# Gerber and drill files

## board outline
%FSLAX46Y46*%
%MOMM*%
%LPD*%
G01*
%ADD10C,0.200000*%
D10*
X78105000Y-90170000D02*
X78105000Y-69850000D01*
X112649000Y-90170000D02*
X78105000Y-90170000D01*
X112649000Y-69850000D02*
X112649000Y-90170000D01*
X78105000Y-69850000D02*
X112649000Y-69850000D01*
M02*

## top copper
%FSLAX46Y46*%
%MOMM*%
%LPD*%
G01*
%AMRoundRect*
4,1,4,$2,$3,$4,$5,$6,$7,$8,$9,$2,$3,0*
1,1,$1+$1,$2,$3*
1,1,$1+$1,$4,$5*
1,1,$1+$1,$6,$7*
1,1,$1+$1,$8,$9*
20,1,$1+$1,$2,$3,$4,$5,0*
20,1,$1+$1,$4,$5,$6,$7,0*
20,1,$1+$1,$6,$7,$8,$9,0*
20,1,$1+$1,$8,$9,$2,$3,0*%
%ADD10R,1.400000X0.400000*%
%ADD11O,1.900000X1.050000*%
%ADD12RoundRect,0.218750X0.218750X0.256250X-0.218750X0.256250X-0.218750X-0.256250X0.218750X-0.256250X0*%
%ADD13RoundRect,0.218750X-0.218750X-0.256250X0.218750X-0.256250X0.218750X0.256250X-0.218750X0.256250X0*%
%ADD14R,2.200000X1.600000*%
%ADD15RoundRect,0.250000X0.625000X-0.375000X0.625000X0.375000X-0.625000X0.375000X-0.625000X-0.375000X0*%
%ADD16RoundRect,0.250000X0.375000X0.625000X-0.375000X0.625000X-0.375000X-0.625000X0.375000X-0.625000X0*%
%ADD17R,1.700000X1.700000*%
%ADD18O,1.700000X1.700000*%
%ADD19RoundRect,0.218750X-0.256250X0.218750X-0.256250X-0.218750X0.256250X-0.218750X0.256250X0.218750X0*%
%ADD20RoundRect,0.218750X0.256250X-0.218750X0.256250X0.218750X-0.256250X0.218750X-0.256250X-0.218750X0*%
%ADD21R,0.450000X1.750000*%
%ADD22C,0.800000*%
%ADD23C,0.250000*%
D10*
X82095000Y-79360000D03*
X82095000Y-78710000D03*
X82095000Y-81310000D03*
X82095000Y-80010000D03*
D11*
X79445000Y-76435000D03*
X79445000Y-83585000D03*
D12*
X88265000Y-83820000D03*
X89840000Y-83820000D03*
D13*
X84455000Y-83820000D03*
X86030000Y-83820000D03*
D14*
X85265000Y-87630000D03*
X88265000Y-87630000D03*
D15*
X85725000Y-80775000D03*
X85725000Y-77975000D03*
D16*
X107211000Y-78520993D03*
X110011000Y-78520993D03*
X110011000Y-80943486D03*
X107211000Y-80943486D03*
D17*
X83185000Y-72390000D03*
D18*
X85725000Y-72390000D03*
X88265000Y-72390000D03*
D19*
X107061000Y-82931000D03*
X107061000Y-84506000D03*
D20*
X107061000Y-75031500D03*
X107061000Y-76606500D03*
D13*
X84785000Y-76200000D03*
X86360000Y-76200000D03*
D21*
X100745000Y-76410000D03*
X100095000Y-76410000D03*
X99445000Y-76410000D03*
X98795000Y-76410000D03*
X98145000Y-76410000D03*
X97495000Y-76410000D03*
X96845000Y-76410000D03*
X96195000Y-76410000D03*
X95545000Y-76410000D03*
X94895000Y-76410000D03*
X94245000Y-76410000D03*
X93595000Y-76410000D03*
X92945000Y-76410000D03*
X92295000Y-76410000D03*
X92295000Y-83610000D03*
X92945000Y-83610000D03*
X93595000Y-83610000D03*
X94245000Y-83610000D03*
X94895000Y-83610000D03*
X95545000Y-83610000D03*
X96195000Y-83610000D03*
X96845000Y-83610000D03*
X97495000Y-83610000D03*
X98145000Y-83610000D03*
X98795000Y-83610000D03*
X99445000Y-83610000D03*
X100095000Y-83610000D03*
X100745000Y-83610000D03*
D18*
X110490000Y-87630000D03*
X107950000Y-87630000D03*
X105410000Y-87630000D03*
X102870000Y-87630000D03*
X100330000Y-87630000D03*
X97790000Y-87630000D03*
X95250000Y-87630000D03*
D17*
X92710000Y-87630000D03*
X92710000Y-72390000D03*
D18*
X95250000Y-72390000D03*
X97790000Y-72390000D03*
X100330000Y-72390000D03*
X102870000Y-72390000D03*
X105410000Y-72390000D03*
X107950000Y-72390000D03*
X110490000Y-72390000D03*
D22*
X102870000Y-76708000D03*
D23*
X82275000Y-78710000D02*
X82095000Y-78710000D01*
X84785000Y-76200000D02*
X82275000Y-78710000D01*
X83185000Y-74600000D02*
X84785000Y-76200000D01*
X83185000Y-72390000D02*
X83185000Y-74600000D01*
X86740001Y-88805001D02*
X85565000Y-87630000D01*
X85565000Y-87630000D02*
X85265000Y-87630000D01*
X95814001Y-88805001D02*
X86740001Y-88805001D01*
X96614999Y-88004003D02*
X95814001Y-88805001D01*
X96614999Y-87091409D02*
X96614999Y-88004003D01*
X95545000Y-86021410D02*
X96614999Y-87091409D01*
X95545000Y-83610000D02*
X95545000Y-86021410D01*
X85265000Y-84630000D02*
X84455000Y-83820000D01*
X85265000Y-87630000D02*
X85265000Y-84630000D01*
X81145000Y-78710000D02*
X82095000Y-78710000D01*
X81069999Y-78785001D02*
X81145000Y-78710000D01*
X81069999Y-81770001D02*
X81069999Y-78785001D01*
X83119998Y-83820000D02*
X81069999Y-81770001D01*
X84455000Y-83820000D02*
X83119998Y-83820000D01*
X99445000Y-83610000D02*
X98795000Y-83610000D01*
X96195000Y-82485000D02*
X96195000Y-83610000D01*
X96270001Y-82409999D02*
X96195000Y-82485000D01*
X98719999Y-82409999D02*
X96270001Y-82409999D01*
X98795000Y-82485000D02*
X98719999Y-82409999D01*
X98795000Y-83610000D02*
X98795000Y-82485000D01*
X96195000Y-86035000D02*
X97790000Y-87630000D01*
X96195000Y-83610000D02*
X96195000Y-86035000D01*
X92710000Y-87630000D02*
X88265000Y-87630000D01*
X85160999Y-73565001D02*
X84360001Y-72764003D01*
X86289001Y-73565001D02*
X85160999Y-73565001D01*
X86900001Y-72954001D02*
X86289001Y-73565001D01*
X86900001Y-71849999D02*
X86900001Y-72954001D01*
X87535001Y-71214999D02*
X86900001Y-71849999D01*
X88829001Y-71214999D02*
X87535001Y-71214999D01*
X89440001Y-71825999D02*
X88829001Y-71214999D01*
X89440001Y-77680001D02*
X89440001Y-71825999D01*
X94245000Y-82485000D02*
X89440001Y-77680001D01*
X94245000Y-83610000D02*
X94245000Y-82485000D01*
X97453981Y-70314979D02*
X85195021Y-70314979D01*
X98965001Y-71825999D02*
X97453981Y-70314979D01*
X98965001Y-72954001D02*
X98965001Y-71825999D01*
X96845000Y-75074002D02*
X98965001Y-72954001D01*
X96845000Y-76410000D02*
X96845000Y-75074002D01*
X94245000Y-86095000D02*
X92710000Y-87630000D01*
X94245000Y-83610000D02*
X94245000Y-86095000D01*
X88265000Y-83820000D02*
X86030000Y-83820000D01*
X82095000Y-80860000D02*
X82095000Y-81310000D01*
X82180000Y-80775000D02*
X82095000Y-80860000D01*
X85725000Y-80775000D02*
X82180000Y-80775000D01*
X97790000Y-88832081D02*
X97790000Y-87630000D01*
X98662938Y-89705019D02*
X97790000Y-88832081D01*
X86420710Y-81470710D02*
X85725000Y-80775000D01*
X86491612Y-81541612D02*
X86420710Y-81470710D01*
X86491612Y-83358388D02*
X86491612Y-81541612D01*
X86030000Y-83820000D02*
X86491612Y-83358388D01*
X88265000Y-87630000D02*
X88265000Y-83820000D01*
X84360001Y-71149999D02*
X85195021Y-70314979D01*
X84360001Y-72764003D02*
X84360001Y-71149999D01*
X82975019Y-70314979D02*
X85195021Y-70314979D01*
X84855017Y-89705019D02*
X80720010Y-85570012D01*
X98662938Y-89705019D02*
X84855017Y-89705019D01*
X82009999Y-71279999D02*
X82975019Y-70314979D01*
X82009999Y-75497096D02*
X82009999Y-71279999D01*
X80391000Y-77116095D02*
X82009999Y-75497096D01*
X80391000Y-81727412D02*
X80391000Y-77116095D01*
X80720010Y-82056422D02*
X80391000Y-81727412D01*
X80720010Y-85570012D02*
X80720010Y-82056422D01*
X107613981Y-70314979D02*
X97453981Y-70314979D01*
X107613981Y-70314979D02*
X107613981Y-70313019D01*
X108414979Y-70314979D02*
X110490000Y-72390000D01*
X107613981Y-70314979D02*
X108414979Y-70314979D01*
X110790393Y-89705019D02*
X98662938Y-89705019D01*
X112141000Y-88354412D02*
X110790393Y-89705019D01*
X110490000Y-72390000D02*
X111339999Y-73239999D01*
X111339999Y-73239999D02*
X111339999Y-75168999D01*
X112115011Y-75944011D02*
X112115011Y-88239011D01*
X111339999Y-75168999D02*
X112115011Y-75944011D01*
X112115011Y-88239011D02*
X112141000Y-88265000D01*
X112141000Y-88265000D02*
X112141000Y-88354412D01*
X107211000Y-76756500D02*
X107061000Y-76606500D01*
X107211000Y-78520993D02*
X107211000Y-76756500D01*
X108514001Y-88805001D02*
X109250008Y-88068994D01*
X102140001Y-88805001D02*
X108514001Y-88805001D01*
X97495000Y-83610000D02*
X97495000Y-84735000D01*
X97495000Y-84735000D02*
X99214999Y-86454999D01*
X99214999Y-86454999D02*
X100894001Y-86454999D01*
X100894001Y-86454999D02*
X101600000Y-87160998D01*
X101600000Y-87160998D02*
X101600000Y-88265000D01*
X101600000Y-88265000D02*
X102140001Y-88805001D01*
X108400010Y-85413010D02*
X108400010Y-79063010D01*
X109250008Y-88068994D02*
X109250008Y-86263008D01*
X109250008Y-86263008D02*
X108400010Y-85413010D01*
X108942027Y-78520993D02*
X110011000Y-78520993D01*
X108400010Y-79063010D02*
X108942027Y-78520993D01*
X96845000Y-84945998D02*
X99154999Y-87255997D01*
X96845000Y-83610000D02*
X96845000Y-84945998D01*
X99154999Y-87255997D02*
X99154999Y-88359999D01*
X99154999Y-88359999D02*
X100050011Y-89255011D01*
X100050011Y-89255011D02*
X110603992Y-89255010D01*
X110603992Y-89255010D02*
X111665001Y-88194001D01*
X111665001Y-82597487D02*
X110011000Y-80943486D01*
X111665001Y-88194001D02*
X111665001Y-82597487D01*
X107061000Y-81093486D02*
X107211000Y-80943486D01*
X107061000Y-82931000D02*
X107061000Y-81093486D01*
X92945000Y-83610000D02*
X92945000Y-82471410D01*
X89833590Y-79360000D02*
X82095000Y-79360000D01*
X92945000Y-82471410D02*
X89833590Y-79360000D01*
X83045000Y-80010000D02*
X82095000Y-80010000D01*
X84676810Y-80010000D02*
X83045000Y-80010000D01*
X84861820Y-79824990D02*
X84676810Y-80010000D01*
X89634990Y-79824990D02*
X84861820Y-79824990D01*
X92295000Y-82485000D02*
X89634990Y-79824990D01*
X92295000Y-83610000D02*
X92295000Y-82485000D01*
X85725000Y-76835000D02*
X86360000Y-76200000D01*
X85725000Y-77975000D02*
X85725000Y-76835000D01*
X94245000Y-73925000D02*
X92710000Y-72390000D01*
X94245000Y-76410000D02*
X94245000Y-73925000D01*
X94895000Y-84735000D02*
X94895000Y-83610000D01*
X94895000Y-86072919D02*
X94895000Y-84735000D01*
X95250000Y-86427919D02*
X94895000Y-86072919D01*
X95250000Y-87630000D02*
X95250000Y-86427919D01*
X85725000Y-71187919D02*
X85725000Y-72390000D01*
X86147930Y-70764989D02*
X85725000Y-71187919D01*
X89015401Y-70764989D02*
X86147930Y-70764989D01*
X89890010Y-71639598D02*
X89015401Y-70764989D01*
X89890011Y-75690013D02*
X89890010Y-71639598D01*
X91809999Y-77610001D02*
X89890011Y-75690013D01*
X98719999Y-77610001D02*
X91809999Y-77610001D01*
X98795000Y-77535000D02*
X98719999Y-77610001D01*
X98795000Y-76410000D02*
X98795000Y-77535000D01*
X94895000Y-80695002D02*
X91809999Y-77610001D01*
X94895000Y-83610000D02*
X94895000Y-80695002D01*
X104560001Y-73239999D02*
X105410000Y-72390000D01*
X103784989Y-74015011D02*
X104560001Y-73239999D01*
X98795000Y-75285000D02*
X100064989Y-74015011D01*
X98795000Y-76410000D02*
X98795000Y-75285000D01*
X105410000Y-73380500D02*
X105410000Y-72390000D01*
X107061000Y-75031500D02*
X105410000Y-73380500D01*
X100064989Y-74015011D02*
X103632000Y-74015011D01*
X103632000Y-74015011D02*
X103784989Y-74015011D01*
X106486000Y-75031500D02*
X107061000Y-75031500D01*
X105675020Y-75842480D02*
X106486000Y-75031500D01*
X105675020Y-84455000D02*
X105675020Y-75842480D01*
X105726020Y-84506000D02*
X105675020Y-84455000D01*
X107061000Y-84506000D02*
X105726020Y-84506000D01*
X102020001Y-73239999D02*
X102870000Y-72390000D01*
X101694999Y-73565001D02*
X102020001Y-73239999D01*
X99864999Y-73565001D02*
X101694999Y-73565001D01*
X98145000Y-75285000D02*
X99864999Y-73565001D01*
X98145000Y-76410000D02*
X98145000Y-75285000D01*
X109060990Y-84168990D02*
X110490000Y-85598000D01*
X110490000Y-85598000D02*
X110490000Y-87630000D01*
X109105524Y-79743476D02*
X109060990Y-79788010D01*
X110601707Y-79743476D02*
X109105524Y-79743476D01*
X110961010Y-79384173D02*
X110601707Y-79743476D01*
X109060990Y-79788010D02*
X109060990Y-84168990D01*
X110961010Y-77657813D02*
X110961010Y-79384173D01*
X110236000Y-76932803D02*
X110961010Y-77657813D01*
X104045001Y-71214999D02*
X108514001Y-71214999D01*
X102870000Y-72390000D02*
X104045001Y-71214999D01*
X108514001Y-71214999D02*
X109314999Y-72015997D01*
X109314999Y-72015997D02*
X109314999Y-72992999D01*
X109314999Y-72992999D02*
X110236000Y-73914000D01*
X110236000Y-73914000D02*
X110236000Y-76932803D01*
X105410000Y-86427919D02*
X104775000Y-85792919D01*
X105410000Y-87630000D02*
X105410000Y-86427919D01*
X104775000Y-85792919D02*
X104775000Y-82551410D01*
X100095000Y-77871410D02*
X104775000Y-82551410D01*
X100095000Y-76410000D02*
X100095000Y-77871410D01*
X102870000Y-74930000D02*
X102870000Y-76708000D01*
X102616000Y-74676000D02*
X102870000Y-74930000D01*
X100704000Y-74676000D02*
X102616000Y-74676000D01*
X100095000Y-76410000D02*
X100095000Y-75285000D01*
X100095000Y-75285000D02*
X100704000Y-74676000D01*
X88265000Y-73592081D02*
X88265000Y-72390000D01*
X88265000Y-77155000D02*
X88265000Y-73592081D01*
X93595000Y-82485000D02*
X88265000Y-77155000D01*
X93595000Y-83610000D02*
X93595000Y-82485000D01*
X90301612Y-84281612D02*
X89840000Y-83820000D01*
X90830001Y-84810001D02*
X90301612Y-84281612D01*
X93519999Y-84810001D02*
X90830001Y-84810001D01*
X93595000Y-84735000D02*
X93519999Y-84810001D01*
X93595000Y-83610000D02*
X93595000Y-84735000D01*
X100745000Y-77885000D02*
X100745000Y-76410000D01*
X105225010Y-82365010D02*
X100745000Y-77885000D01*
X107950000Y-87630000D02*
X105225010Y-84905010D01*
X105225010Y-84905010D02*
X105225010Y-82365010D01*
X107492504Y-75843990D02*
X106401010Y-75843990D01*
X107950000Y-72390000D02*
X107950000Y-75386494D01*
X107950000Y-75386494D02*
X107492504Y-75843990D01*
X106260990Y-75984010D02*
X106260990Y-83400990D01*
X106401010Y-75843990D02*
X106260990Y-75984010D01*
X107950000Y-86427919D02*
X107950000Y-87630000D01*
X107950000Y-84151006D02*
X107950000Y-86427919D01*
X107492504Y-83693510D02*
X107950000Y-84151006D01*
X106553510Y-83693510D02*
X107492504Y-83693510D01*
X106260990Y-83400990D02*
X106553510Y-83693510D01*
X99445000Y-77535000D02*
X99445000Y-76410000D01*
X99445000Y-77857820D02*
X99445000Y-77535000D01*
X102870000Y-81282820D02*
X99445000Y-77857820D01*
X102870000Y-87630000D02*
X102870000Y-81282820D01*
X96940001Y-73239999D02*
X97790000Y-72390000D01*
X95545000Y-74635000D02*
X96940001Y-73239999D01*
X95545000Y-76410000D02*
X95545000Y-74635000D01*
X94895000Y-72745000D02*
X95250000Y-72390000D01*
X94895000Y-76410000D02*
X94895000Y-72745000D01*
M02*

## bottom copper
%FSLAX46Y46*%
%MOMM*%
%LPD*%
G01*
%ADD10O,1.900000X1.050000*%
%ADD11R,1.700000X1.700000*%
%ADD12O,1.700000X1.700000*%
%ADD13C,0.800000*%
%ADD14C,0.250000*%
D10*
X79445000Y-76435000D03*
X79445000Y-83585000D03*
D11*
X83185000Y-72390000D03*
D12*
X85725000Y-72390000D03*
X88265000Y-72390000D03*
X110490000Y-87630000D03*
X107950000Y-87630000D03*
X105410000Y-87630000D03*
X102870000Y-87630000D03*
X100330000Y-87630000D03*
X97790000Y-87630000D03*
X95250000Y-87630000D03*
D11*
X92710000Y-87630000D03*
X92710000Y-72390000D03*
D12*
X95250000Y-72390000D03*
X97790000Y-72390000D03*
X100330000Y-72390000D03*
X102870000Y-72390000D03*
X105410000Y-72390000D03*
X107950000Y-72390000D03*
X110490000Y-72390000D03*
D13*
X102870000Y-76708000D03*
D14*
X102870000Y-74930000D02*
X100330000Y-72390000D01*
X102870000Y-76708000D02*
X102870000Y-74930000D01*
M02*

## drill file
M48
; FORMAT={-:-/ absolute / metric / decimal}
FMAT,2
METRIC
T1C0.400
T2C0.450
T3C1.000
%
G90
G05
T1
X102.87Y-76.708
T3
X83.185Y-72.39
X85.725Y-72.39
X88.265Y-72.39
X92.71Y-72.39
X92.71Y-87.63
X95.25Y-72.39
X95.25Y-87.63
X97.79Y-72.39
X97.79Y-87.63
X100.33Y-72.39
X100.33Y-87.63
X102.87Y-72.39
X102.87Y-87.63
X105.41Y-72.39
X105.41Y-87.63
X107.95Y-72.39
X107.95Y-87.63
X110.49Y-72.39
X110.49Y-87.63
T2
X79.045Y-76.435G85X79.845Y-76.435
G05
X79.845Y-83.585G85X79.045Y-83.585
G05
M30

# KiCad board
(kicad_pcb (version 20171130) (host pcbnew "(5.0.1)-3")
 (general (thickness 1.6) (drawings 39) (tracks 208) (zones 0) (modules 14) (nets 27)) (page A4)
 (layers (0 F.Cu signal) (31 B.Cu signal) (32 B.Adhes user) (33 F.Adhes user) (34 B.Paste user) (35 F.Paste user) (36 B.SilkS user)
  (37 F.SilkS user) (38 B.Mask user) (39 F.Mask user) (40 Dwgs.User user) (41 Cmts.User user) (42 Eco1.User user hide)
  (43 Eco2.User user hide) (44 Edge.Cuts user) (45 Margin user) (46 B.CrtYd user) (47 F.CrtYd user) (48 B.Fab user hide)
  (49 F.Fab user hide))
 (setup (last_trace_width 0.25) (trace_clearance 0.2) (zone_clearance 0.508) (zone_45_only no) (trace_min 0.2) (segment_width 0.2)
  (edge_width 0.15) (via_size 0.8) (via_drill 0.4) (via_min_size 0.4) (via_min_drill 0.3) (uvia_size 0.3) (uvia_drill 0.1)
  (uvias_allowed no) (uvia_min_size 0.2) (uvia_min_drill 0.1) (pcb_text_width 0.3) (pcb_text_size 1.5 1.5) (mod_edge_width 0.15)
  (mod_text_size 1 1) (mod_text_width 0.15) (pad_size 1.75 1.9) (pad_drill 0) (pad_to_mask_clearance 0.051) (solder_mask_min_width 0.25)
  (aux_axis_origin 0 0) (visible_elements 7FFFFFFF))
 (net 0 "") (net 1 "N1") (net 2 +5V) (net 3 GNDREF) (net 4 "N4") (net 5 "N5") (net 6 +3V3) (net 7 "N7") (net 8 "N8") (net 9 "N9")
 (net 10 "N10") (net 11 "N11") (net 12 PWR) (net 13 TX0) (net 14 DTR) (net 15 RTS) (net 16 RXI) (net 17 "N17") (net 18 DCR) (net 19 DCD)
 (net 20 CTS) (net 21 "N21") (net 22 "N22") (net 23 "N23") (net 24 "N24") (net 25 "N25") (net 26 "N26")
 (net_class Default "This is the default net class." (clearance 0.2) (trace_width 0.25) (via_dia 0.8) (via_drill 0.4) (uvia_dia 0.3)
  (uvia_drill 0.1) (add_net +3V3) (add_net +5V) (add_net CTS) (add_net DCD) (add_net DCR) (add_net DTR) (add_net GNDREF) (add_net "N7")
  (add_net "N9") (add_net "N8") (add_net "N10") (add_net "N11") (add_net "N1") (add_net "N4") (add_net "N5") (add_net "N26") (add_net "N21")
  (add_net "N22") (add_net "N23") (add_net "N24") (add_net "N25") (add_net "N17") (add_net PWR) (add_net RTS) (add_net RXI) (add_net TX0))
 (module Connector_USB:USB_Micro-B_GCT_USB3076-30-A (layer F.Cu) (at 80.645 80.01 270)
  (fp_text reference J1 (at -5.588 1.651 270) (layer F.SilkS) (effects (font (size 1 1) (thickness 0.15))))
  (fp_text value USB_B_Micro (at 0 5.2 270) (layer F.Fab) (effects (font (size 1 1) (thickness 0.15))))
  (pad 2 smd rect (at -0.65 -1.45 270) (size 0.4 1.4) (layers F.Cu F.Paste F.Mask) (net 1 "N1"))
  (pad 1 smd rect (at -1.3 -1.45 270) (size 0.4 1.4) (layers F.Cu F.Paste F.Mask) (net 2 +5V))
  (pad 5 smd rect (at 1.3 -1.45 270) (size 0.4 1.4) (layers F.Cu F.Paste F.Mask) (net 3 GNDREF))
  (pad 3 smd rect (at 0 -1.45 270) (size 0.4 1.4) (layers F.Cu F.Paste F.Mask) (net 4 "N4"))
  (pad 6 thru_hole oval (at -3.575 1.2 90) (size 1.05 1.9) (drill oval 0.45 1.25) (layers *.Cu *.Mask) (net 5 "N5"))
  (pad 6 thru_hole oval (at 3.575 1.2 270) (size 1.05 1.9) (drill oval 0.45 1.25) (layers *.Cu *.Mask) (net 5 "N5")))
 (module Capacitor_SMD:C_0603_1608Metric (layer F.Cu) (at 89.0525 83.82 180)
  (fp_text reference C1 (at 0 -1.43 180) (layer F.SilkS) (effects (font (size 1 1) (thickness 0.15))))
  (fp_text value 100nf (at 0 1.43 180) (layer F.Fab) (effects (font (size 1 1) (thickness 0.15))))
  (pad 2 smd roundrect (at 0.7875 0 180) (size 0.875 0.95) (layers F.Cu F.Paste F.Mask) (roundrect_rratio 0.25) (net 3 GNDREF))
  (pad 1 smd roundrect (at -0.7875 0 180) (size 0.875 0.95) (layers F.Cu F.Paste F.Mask) (roundrect_rratio 0.25) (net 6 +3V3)))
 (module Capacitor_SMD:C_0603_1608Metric (layer F.Cu) (at 85.2425 83.82)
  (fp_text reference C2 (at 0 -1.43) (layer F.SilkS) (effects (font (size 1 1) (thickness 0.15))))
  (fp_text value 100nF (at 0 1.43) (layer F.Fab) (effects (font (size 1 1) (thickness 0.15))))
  (pad 1 smd roundrect (at -0.7875 0) (size 0.875 0.95) (layers F.Cu F.Paste F.Mask) (roundrect_rratio 0.25) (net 2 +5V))
  (pad 2 smd roundrect (at 0.7875 0) (size 0.875 0.95) (layers F.Cu F.Paste F.Mask) (roundrect_rratio 0.25) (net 3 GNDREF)))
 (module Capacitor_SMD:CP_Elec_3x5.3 (layer F.Cu) (at 86.765 87.63)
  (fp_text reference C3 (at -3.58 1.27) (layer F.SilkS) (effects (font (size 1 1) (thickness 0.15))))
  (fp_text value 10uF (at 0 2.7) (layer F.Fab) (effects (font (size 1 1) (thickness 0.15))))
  (pad 1 smd rect (at -1.5 0) (size 2.2 1.6) (layers F.Cu F.Paste F.Mask) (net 2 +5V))
  (pad 2 smd rect (at 1.5 0) (size 2.2 1.6) (layers F.Cu F.Paste F.Mask) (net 3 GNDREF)))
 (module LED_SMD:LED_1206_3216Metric (layer F.Cu) (at 85.725 79.375 90)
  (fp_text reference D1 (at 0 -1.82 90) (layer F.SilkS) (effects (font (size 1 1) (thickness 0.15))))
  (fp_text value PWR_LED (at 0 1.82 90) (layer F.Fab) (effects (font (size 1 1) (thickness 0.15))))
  (pad 1 smd roundrect (at -1.4 0 90) (size 1.25 1.75) (layers F.Cu F.Paste F.Mask) (roundrect_rratio 0.2) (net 3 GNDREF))
  (pad 2 smd roundrect (at 1.4 0 90) (size 1.25 1.75) (layers F.Cu F.Paste F.Mask) (roundrect_rratio 0.2) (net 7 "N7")))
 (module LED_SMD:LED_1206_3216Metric (layer F.Cu) (at 108.611 78.520993 180)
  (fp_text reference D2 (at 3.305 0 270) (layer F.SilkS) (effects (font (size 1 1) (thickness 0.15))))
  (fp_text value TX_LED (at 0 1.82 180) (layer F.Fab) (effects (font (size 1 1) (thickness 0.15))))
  (pad 2 smd roundrect (at 1.4 0 180) (size 1.25 1.75) (layers F.Cu F.Paste F.Mask) (roundrect_rratio 0.2) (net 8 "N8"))
  (pad 1 smd roundrect (at -1.4 0 180) (size 1.25 1.75) (layers F.Cu F.Paste F.Mask) (roundrect_rratio 0.2) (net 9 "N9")))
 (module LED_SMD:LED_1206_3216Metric (layer F.Cu) (at 108.611 80.943486 180)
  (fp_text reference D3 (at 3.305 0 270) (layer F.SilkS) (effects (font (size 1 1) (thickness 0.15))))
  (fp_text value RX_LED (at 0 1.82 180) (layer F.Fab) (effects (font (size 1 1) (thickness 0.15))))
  (pad 1 smd roundrect (at -1.4 0 180) (size 1.25 1.75) (layers F.Cu F.Paste F.Mask) (roundrect_rratio 0.2) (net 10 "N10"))
  (pad 2 smd roundrect (at 1.4 0 180) (size 1.25 1.75) (layers F.Cu F.Paste F.Mask) (roundrect_rratio 0.2) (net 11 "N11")))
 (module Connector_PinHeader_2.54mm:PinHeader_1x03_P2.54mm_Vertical (layer F.Cu) (at 83.185 72.39 90)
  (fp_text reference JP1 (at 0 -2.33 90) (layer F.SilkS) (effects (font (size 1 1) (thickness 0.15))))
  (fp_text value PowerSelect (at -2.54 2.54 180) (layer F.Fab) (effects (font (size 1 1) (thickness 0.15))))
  (pad 1 thru_hole rect (at 0 0 90) (size 1.7 1.7) (drill 1) (layers *.Cu *.Mask) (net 2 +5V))
  (pad 2 thru_hole oval (at 0 2.54 90) (size 1.7 1.7) (drill 1) (layers *.Cu *.Mask) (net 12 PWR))
  (pad 3 thru_hole oval (at 0 5.08 90) (size 1.7 1.7) (drill 1) (layers *.Cu *.Mask) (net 6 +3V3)))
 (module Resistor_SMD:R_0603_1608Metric (layer F.Cu) (at 107.061 83.7185 270)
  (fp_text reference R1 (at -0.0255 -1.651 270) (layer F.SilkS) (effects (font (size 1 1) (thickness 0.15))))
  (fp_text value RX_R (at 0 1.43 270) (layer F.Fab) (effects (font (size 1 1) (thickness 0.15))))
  (pad 1 smd roundrect (at -0.7875 0 270) (size 0.875 0.95) (layers F.Cu F.Paste F.Mask) (roundrect_rratio 0.25) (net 11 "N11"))
  (pad 2 smd roundrect (at 0.7875 0 270) (size 0.875 0.95) (layers F.Cu F.Paste F.Mask) (roundrect_rratio 0.25) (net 12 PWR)))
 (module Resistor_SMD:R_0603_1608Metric (layer F.Cu) (at 107.061 75.819 90)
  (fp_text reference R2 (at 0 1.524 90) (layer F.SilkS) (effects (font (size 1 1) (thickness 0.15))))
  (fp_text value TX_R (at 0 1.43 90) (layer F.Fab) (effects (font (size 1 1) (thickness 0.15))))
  (pad 2 smd roundrect (at 0.7875 0 90) (size 0.875 0.95) (layers F.Cu F.Paste F.Mask) (roundrect_rratio 0.25) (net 12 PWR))
  (pad 1 smd roundrect (at -0.7875 0 90) (size 0.875 0.95) (layers F.Cu F.Paste F.Mask) (roundrect_rratio 0.25) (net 8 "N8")))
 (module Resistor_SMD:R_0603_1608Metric (layer F.Cu) (at 85.5725 76.2)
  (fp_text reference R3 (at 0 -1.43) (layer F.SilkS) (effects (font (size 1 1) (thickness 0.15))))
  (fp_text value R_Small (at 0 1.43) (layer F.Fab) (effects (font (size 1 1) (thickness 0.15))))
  (pad 1 smd roundrect (at -0.7875 0) (size 0.875 0.95) (layers F.Cu F.Paste F.Mask) (roundrect_rratio 0.25) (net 2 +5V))
  (pad 2 smd roundrect (at 0.7875 0) (size 0.875 0.95) (layers F.Cu F.Paste F.Mask) (roundrect_rratio 0.25) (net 7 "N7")))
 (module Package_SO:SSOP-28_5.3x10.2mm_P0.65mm (layer F.Cu) (at 96.52 80.01 270)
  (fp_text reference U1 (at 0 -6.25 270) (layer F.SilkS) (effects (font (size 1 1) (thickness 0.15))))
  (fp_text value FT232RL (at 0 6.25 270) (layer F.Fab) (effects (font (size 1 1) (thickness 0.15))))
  (pad 1 smd rect (at -3.6 -4.225 270) (size 1.75 0.45) (layers F.Cu F.Paste F.Mask) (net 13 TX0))
  (pad 2 smd rect (at -3.6 -3.575 270) (size 1.75 0.45) (layers F.Cu F.Paste F.Mask) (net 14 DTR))
  (pad 3 smd rect (at -3.6 -2.925 270) (size 1.75 0.45) (layers F.Cu F.Paste F.Mask) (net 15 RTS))
  (pad 4 smd rect (at -3.6 -2.275 270) (size 1.75 0.45) (layers F.Cu F.Paste F.Mask) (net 12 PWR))
  (pad 5 smd rect (at -3.6 -1.625 270) (size 1.75 0.45) (layers F.Cu F.Paste F.Mask) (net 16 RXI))
  (pad 6 smd rect (at -3.6 -0.975 270) (size 1.75 0.45) (layers F.Cu F.Paste F.Mask) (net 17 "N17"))
  (pad 7 smd rect (at -3.6 -0.325 270) (size 1.75 0.45) (layers F.Cu F.Paste F.Mask) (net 3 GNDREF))
  (pad 8 smd rect (at -3.6 0.325 270) (size 1.75 0.45) (layers F.Cu F.Paste F.Mask))
  (pad 9 smd rect (at -3.6 0.975 270) (size 1.75 0.45) (layers F.Cu F.Paste F.Mask) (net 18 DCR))
  (pad 10 smd rect (at -3.6 1.625 270) (size 1.75 0.45) (layers F.Cu F.Paste F.Mask) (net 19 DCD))
  (pad 11 smd rect (at -3.6 2.275 270) (size 1.75 0.45) (layers F.Cu F.Paste F.Mask) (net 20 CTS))
  (pad 12 smd rect (at -3.6 2.925 270) (size 1.75 0.45) (layers F.Cu F.Paste F.Mask) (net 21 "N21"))
  (pad 13 smd rect (at -3.6 3.575 270) (size 1.75 0.45) (layers F.Cu F.Paste F.Mask) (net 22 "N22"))
  (pad 14 smd rect (at -3.6 4.225 270) (size 1.75 0.45) (layers F.Cu F.Paste F.Mask) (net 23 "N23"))
  (pad 15 smd rect (at 3.6 4.225 270) (size 1.75 0.45) (layers F.Cu F.Paste F.Mask) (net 4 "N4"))
  (pad 16 smd rect (at 3.6 3.575 270) (size 1.75 0.45) (layers F.Cu F.Paste F.Mask) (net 1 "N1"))
  (pad 17 smd rect (at 3.6 2.925 270) (size 1.75 0.45) (layers F.Cu F.Paste F.Mask) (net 6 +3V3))
  (pad 18 smd rect (at 3.6 2.275 270) (size 1.75 0.45) (layers F.Cu F.Paste F.Mask) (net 3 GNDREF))
  (pad 19 smd rect (at 3.6 1.625 270) (size 1.75 0.45) (layers F.Cu F.Paste F.Mask) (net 12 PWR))
  (pad 20 smd rect (at 3.6 0.975 270) (size 1.75 0.45) (layers F.Cu F.Paste F.Mask) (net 2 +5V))
  (pad 21 smd rect (at 3.6 0.325 270) (size 1.75 0.45) (layers F.Cu F.Paste F.Mask) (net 3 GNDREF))
  (pad 22 smd rect (at 3.6 -0.325 270) (size 1.75 0.45) (layers F.Cu F.Paste F.Mask) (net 10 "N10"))
  (pad 23 smd rect (at 3.6 -0.975 270) (size 1.75 0.45) (layers F.Cu F.Paste F.Mask) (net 9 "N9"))
  (pad 24 smd rect (at 3.6 -1.625 270) (size 1.75 0.45) (layers F.Cu F.Paste F.Mask))
  (pad 25 smd rect (at 3.6 -2.275 270) (size 1.75 0.45) (layers F.Cu F.Paste F.Mask) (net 3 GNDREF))
  (pad 26 smd rect (at 3.6 -2.925 270) (size 1.75 0.45) (layers F.Cu F.Paste F.Mask) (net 3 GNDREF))
  (pad 27 smd rect (at 3.6 -3.575 270) (size 1.75 0.45) (layers F.Cu F.Paste F.Mask) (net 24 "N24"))
  (pad 28 smd rect (at 3.6 -4.225 270) (size 1.75 0.45) (layers F.Cu F.Paste F.Mask) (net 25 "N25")))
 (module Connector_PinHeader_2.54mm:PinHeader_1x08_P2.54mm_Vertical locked (layer F.Cu) (at 92.71 87.63 90)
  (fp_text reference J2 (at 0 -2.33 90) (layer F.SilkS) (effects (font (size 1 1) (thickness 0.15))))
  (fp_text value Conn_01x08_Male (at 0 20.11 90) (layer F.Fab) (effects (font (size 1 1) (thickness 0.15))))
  (pad 8 thru_hole oval (at 0 17.78 90) (size 1.7 1.7) (drill 1) (layers *.Cu *.Mask) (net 16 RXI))
  (pad 7 thru_hole oval (at 0 15.24 90) (size 1.7 1.7) (drill 1) (layers *.Cu *.Mask) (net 13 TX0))
  (pad 6 thru_hole oval (at 0 12.7 90) (size 1.7 1.7) (drill 1) (layers *.Cu *.Mask) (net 14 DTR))
  (pad 5 thru_hole oval (at 0 10.16 90) (size 1.7 1.7) (drill 1) (layers *.Cu *.Mask) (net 15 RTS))
  (pad 4 thru_hole oval (at 0 7.62 90) (size 1.7 1.7) (drill 1) (layers *.Cu *.Mask) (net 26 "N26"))
  (pad 3 thru_hole oval (at 0 5.08 90) (size 1.7 1.7) (drill 1) (layers *.Cu *.Mask) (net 3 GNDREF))
  (pad 2 thru_hole oval (at 0 2.54 90) (size 1.7 1.7) (drill 1) (layers *.Cu *.Mask) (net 12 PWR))
  (pad 1 thru_hole rect (at 0 0 90) (size 1.7 1.7) (drill 1) (layers *.Cu *.Mask) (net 3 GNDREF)))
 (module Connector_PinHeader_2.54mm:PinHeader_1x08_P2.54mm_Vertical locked (layer F.Cu) (at 92.71 72.39 90)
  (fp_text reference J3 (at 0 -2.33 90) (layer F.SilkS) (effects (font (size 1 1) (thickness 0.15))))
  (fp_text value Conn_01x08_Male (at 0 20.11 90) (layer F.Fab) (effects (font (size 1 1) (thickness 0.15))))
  (pad 1 thru_hole rect (at 0 0 90) (size 1.7 1.7) (drill 1) (layers *.Cu *.Mask) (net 20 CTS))
  (pad 2 thru_hole oval (at 0 2.54 90) (size 1.7 1.7) (drill 1) (layers *.Cu *.Mask) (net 19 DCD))
  (pad 3 thru_hole oval (at 0 5.08 90) (size 1.7 1.7) (drill 1) (layers *.Cu *.Mask) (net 18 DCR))
  (pad 4 thru_hole oval (at 0 7.62 90) (size 1.7 1.7) (drill 1) (layers *.Cu *.Mask) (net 14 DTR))
  (pad 5 thru_hole oval (at 0 10.16 90) (size 1.7 1.7) (drill 1) (layers *.Cu *.Mask) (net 16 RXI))
  (pad 6 thru_hole oval (at 0 12.7 90) (size 1.7 1.7) (drill 1) (layers *.Cu *.Mask) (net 12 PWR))
  (pad 7 thru_hole oval (at 0 15.24 90) (size 1.7 1.7) (drill 1) (layers *.Cu *.Mask) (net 13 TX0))
  (pad 8 thru_hole oval (at 0 17.78 90) (size 1.7 1.7) (drill 1) (layers *.Cu *.Mask) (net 3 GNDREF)))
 (gr_line (start 78.105 90.17) (end 78.105 69.85) (layer Edge.Cuts) (width 0.2))
 (gr_line (start 112.649 90.17) (end 78.105 90.17) (layer Edge.Cuts) (width 0.2))
 (gr_line (start 112.649 69.85) (end 112.649 90.17) (layer Edge.Cuts) (width 0.2))
 (gr_line (start 78.105 69.85) (end 112.649 69.85) (layer Edge.Cuts) (width 0.2))
 (via (at 102.87 76.708) (size 0.8) (drill 0.4) (layers F.Cu B.Cu) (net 14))
 (segment (start 82.275 78.71) (end 82.095 78.71) (width 0.25) (layer F.Cu) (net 2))
 (segment (start 84.785 76.2) (end 82.275 78.71) (width 0.25) (layer F.Cu) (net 2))
 (segment (start 83.185 74.6) (end 84.785 76.2) (width 0.25) (layer F.Cu) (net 2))
 (segment (start 83.185 72.39) (end 83.185 74.6) (width 0.25) (layer F.Cu) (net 2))
 (segment (start 86.740001 88.805001) (end 85.565 87.63) (width 0.25) (layer F.Cu) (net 2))
 (segment (start 85.565 87.63) (end 85.265 87.63) (width 0.25) (layer F.Cu) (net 2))
 (segment (start 95.814001 88.805001) (end 86.740001 88.805001) (width 0.25) (layer F.Cu) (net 2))
 (segment (start 96.614999 88.004003) (end 95.814001 88.805001) (width 0.25) (layer F.Cu) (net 2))
 (segment (start 96.614999 87.091409) (end 96.614999 88.004003) (width 0.25) (layer F.Cu) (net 2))
 (segment (start 95.545 86.02141) (end 96.614999 87.091409) (width 0.25) (layer F.Cu) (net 2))
 (segment (start 95.545 83.61) (end 95.545 86.02141) (width 0.25) (layer F.Cu) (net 2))
 (segment (start 85.265 84.63) (end 84.455 83.82) (width 0.25) (layer F.Cu) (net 2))
 (segment (start 85.265 87.63) (end 85.265 84.63) (width 0.25) (layer F.Cu) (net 2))
 (segment (start 81.145 78.71) (end 82.095 78.71) (width 0.25) (layer F.Cu) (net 2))
 (segment (start 81.069999 78.785001) (end 81.145 78.71) (width 0.25) (layer F.Cu) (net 2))
 (segment (start 81.069999 81.770001) (end 81.069999 78.785001) (width 0.25) (layer F.Cu) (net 2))
 (segment (start 83.119998 83.82) (end 81.069999 81.770001) (width 0.25) (layer F.Cu) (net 2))
 (segment (start 84.455 83.82) (end 83.119998 83.82) (width 0.25) (layer F.Cu) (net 2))
 (segment (start 99.445 83.61) (end 98.795 83.61) (width 0.25) (layer F.Cu) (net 3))
 (segment (start 96.195 82.485) (end 96.195 83.61) (width 0.25) (layer F.Cu) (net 3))
 (segment (start 96.270001 82.409999) (end 96.195 82.485) (width 0.25) (layer F.Cu) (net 3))
 (segment (start 98.719999 82.409999) (end 96.270001 82.409999) (width 0.25) (layer F.Cu) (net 3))
 (segment (start 98.795 82.485) (end 98.719999 82.409999) (width 0.25) (layer F.Cu) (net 3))
 (segment (start 98.795 83.61) (end 98.795 82.485) (width 0.25) (layer F.Cu) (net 3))
 (segment (start 96.195 86.035) (end 97.79 87.63) (width 0.25) (layer F.Cu) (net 3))
 (segment (start 96.195 83.61) (end 96.195 86.035) (width 0.25) (layer F.Cu) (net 3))
 (segment (start 92.71 87.63) (end 88.265 87.63) (width 0.25) (layer F.Cu) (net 3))
 (segment (start 85.160999 73.565001) (end 84.360001 72.764003) (width 0.25) (layer F.Cu) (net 3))
 (segment (start 86.289001 73.565001) (end 85.160999 73.565001) (width 0.25) (layer F.Cu) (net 3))
 (segment (start 86.900001 72.954001) (end 86.289001 73.565001) (width 0.25) (layer F.Cu) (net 3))
 (segment (start 86.900001 71.849999) (end 86.900001 72.954001) (width 0.25) (layer F.Cu) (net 3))
 (segment (start 87.535001 71.214999) (end 86.900001 71.849999) (width 0.25) (layer F.Cu) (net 3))
 (segment (start 88.829001 71.214999) (end 87.535001 71.214999) (width 0.25) (layer F.Cu) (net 3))
 (segment (start 89.440001 71.825999) (end 88.829001 71.214999) (width 0.25) (layer F.Cu) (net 3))
 (segment (start 89.440001 77.680001) (end 89.440001 71.825999) (width 0.25) (layer F.Cu) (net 3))
 (segment (start 94.245 82.485) (end 89.440001 77.680001) (width 0.25) (layer F.Cu) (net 3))
 (segment (start 94.245 83.61) (end 94.245 82.485) (width 0.25) (layer F.Cu) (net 3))
 (segment (start 97.453981 70.314979) (end 85.195021 70.314979) (width 0.25) (layer F.Cu) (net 3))
 (segment (start 98.965001 71.825999) (end 97.453981 70.314979) (width 0.25) (layer F.Cu) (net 3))
 (segment (start 98.965001 72.954001) (end 98.965001 71.825999) (width 0.25) (layer F.Cu) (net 3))
 (segment (start 96.845 75.074002) (end 98.965001 72.954001) (width 0.25) (layer F.Cu) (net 3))
 (segment (start 96.845 76.41) (end 96.845 75.074002) (width 0.25) (layer F.Cu) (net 3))
 (segment (start 94.245 86.095) (end 92.71 87.63) (width 0.25) (layer F.Cu) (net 3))
 (segment (start 94.245 83.61) (end 94.245 86.095) (width 0.25) (layer F.Cu) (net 3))
 (segment (start 88.265 83.82) (end 86.03 83.82) (width 0.25) (layer F.Cu) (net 3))
 (segment (start 82.095 80.86) (end 82.095 81.31) (width 0.25) (layer F.Cu) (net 3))
 (segment (start 82.18 80.775) (end 82.095 80.86) (width 0.25) (layer F.Cu) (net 3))
 (segment (start 85.725 80.775) (end 82.18 80.775) (width 0.25) (layer F.Cu) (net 3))
 (segment (start 97.79 88.832081) (end 97.79 87.63) (width 0.25) (layer F.Cu) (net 3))
 (segment (start 98.662938 89.705019) (end 97.79 88.832081) (width 0.25) (layer F.Cu) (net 3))
 (segment (start 86.42071 81.47071) (end 85.725 80.775) (width 0.25) (layer F.Cu) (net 3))
 (segment (start 86.491612 81.541612) (end 86.42071 81.47071) (width 0.25) (layer F.Cu) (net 3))
 (segment (start 86.491612 83.358388) (end 86.491612 81.541612) (width 0.25) (layer F.Cu) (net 3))
 (segment (start 86.03 83.82) (end 86.491612 83.358388) (width 0.25) (layer F.Cu) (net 3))
 (segment (start 88.265 87.63) (end 88.265 83.82) (width 0.25) (layer F.Cu) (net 3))
 (segment (start 84.360001 71.149999) (end 85.195021 70.314979) (width 0.25) (layer F.Cu) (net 3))
 (segment (start 84.360001 72.764003) (end 84.360001 71.149999) (width 0.25) (layer F.Cu) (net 3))
 (segment (start 82.975019 70.314979) (end 85.195021 70.314979) (width 0.25) (layer F.Cu) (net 3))
 (segment (start 84.855017 89.705019) (end 80.72001 85.570012) (width 0.25) (layer F.Cu) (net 3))
 (segment (start 98.662938 89.705019) (end 84.855017 89.705019) (width 0.25) (layer F.Cu) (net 3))
 (segment (start 82.009999 71.279999) (end 82.975019 70.314979) (width 0.25) (layer F.Cu) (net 3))
 (segment (start 82.009999 75.497096) (end 82.009999 71.279999) (width 0.25) (layer F.Cu) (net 3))
 (segment (start 80.391 77.116095) (end 82.009999 75.497096) (width 0.25) (layer F.Cu) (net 3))
 (segment (start 80.391 81.727412) (end 80.391 77.116095) (width 0.25) (layer F.Cu) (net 3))
 (segment (start 80.72001 82.056422) (end 80.391 81.727412) (width 0.25) (layer F.Cu) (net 3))
 (segment (start 80.72001 85.570012) (end 80.72001 82.056422) (width 0.25) (layer F.Cu) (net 3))
 (segment (start 107.613981 70.314979) (end 97.453981 70.314979) (width 0.25) (layer F.Cu) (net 3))
 (segment (start 107.613981 70.314979) (end 107.613981 70.313019) (width 0.25) (layer F.Cu) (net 3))
 (segment (start 108.414979 70.314979) (end 110.49 72.39) (width 0.25) (layer F.Cu) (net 3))
 (segment (start 107.613981 70.314979) (end 108.414979 70.314979) (width 0.25) (layer F.Cu) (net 3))
 (segment (start 110.790393 89.705019) (end 98.662938 89.705019) (width 0.25) (layer F.Cu) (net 3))
 (segment (start 112.141 88.354412) (end 110.790393 89.705019) (width 0.25) (layer F.Cu) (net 3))
 (segment (start 110.49 72.39) (end 111.339999 73.239999) (width 0.25) (layer F.Cu) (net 3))
 (segment (start 111.339999 73.239999) (end 111.339999 75.168999) (width 0.25) (layer F.Cu) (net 3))
 (segment (start 112.115011 75.944011) (end 112.115011 88.239011) (width 0.25) (layer F.Cu) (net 3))
 (segment (start 111.339999 75.168999) (end 112.115011 75.944011) (width 0.25) (layer F.Cu) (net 3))
 (segment (start 112.115011 88.239011) (end 112.141 88.265) (width 0.25) (layer F.Cu) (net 3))
 (segment (start 112.141 88.265) (end 112.141 88.354412) (width 0.25) (layer F.Cu) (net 3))
 (segment (start 107.211 76.7565) (end 107.061 76.6065) (width 0.25) (layer F.Cu) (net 8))
 (segment (start 107.211 78.520993) (end 107.211 76.7565) (width 0.25) (layer F.Cu) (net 8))
 (segment (start 108.514001 88.805001) (end 109.250008 88.068994) (width 0.25) (layer F.Cu) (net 9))
 (segment (start 102.140001 88.805001) (end 108.514001 88.805001) (width 0.25) (layer F.Cu) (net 9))
 (segment (start 97.495 83.61) (end 97.495 84.735) (width 0.25) (layer F.Cu) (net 9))
 (segment (start 97.495 84.735) (end 99.214999 86.454999) (width 0.25) (layer F.Cu) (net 9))
 (segment (start 99.214999 86.454999) (end 100.894001 86.454999) (width 0.25) (layer F.Cu) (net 9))
 (segment (start 100.894001 86.454999) (end 101.6 87.160998) (width 0.25) (layer F.Cu) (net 9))
 (segment (start 101.6 87.160998) (end 101.6 88.265) (width 0.25) (layer F.Cu) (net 9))
 (segment (start 101.6 88.265) (end 102.140001 88.805001) (width 0.25) (layer F.Cu) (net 9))
 (segment (start 108.40001 85.41301) (end 108.40001 79.06301) (width 0.25) (layer F.Cu) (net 9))
 (segment (start 109.250008 88.068994) (end 109.250008 86.263008) (width 0.25) (layer F.Cu) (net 9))
 (segment (start 109.250008 86.263008) (end 108.40001 85.41301) (width 0.25) (layer F.Cu) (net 9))
 (segment (start 108.942027 78.520993) (end 110.011 78.520993) (width 0.25) (layer F.Cu) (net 9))
 (segment (start 108.40001 79.06301) (end 108.942027 78.520993) (width 0.25) (layer F.Cu) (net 9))
 (segment (start 96.845 84.945998) (end 99.154999 87.255997) (width 0.25) (layer F.Cu) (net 10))
 (segment (start 96.845 83.61) (end 96.845 84.945998) (width 0.25) (layer F.Cu) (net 10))
 (segment (start 99.154999 87.255997) (end 99.154999 88.359999) (width 0.25) (layer F.Cu) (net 10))
 (segment (start 99.154999 88.359999) (end 100.050011 89.255011) (width 0.25) (layer F.Cu) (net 10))
 (segment (start 100.050011 89.255011) (end 110.603992 89.25501) (width 0.25) (layer F.Cu) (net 10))
 (segment (start 110.603992 89.25501) (end 111.665001 88.194001) (width 0.25) (layer F.Cu) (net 10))
 (segment (start 111.665001 82.597487) (end 110.011 80.943486) (width 0.25) (layer F.Cu) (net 10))
 (segment (start 111.665001 88.194001) (end 111.665001 82.597487) (width 0.25) (layer F.Cu) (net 10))
 (segment (start 107.061 81.093486) (end 107.211 80.943486) (width 0.25) (layer F.Cu) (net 11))
 (segment (start 107.061 82.931) (end 107.061 81.093486) (width 0.25) (layer F.Cu) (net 11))
 (segment (start 92.945 83.61) (end 92.945 82.47141) (width 0.25) (layer F.Cu) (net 1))
 (segment (start 89.83359 79.36) (end 82.095 79.36) (width 0.25) (layer F.Cu) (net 1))
 (segment (start 92.945 82.47141) (end 89.83359 79.36) (width 0.25) (layer F.Cu) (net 1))
 (segment (start 83.045 80.01) (end 82.095 80.01) (width 0.25) (layer F.Cu) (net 4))
 (segment (start 84.67681 80.01) (end 83.045 80.01) (width 0.25) (layer F.Cu) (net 4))
 (segment (start 84.86182 79.82499) (end 84.67681 80.01) (width 0.25) (layer F.Cu) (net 4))
 (segment (start 89.63499 79.82499) (end 84.86182 79.82499) (width 0.25) (layer F.Cu) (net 4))
 (segment (start 92.295 82.485) (end 89.63499 79.82499) (width 0.25) (layer F.Cu) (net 4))
 (segment (start 92.295 83.61) (end 92.295 82.485) (width 0.25) (layer F.Cu) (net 4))
 (segment (start 85.725 76.835) (end 86.36 76.2) (width 0.25) (layer F.Cu) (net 7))
 (segment (start 85.725 77.975) (end 85.725 76.835) (width 0.25) (layer F.Cu) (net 7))
 (segment (start 94.245 73.925) (end 92.71 72.39) (width 0.25) (layer F.Cu) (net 20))
 (segment (start 94.245 76.41) (end 94.245 73.925) (width 0.25) (layer F.Cu) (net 20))
 (segment (start 94.895 84.735) (end 94.895 83.61) (width 0.25) (layer F.Cu) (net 12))
 (segment (start 94.895 86.072919) (end 94.895 84.735) (width 0.25) (layer F.Cu) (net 12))
 (segment (start 95.25 86.427919) (end 94.895 86.072919) (width 0.25) (layer F.Cu) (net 12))
 (segment (start 95.25 87.63) (end 95.25 86.427919) (width 0.25) (layer F.Cu) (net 12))
 (segment (start 85.725 71.187919) (end 85.725 72.39) (width 0.25) (layer F.Cu) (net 12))
 (segment (start 86.14793 70.764989) (end 85.725 71.187919) (width 0.25) (layer F.Cu) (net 12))
 (segment (start 89.015401 70.764989) (end 86.14793 70.764989) (width 0.25) (layer F.Cu) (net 12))
 (segment (start 89.89001 71.639598) (end 89.015401 70.764989) (width 0.25) (layer F.Cu) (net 12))
 (segment (start 89.890011 75.690013) (end 89.89001 71.639598) (width 0.25) (layer F.Cu) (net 12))
 (segment (start 91.809999 77.610001) (end 89.890011 75.690013) (width 0.25) (layer F.Cu) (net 12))
 (segment (start 98.719999 77.610001) (end 91.809999 77.610001) (width 0.25) (layer F.Cu) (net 12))
 (segment (start 98.795 77.535) (end 98.719999 77.610001) (width 0.25) (layer F.Cu) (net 12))
 (segment (start 98.795 76.41) (end 98.795 77.535) (width 0.25) (layer F.Cu) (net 12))
 (segment (start 94.895 80.695002) (end 91.809999 77.610001) (width 0.25) (layer F.Cu) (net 12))
 (segment (start 94.895 83.61) (end 94.895 80.695002) (width 0.25) (layer F.Cu) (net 12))
 (segment (start 104.560001 73.239999) (end 105.41 72.39) (width 0.25) (layer F.Cu) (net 12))
 (segment (start 103.784989 74.015011) (end 104.560001 73.239999) (width 0.25) (layer F.Cu) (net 12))
 (segment (start 98.795 75.285) (end 100.064989 74.015011) (width 0.25) (layer F.Cu) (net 12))
 (segment (start 98.795 76.41) (end 98.795 75.285) (width 0.25) (layer F.Cu) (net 12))
 (segment (start 105.41 73.3805) (end 105.41 72.39) (width 0.25) (layer F.Cu) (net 12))
 (segment (start 107.061 75.0315) (end 105.41 73.3805) (width 0.25) (layer F.Cu) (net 12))
 (segment (start 100.064989 74.015011) (end 103.632 74.015011) (width 0.25) (layer F.Cu) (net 12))
 (segment (start 103.632 74.015011) (end 103.784989 74.015011) (width 0.25) (layer F.Cu) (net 12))
 (segment (start 106.486 75.0315) (end 107.061 75.0315) (width 0.25) (layer F.Cu) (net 12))
 (segment (start 105.67502 75.84248) (end 106.486 75.0315) (width 0.25) (layer F.Cu) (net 12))
 (segment (start 105.67502 84.455) (end 105.67502 75.84248) (width 0.25) (layer F.Cu) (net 12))
 (segment (start 105.72602 84.506) (end 105.67502 84.455) (width 0.25) (layer F.Cu) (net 12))
 (segment (start 107.061 84.506) (end 105.72602 84.506) (width 0.25) (layer F.Cu) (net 12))
 (segment (start 102.020001 73.239999) (end 102.87 72.39) (width 0.25) (layer F.Cu) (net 16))
 (segment (start 101.694999 73.565001) (end 102.020001 73.239999) (width 0.25) (layer F.Cu) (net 16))
 (segment (start 99.864999 73.565001) (end 101.694999 73.565001) (width 0.25) (layer F.Cu) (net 16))
 (segment (start 98.145 75.285) (end 99.864999 73.565001) (width 0.25) (layer F.Cu) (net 16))
 (segment (start 98.145 76.41) (end 98.145 75.285) (width 0.25) (layer F.Cu) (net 16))
 (segment (start 109.06099 84.16899) (end 110.49 85.598) (width 0.25) (layer F.Cu) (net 16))
 (segment (start 110.49 85.598) (end 110.49 87.63) (width 0.25) (layer F.Cu) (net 16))
 (segment (start 109.105524 79.743476) (end 109.06099 79.78801) (width 0.25) (layer F.Cu) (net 16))
 (segment (start 110.601707 79.743476) (end 109.105524 79.743476) (width 0.25) (layer F.Cu) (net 16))
 (segment (start 110.96101 79.384173) (end 110.601707 79.743476) (width 0.25) (layer F.Cu) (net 16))
 (segment (start 109.06099 79.78801) (end 109.06099 84.16899) (width 0.25) (layer F.Cu) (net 16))
 (segment (start 110.96101 77.657813) (end 110.96101 79.384173) (width 0.25) (layer F.Cu) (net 16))
 (segment (start 110.236 76.932803) (end 110.96101 77.657813) (width 0.25) (layer F.Cu) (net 16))
 (segment (start 104.045001 71.214999) (end 108.514001 71.214999) (width 0.25) (layer F.Cu) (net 16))
 (segment (start 102.87 72.39) (end 104.045001 71.214999) (width 0.25) (layer F.Cu) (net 16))
 (segment (start 108.514001 71.214999) (end 109.314999 72.015997) (width 0.25) (layer F.Cu) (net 16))
 (segment (start 109.314999 72.015997) (end 109.314999 72.992999) (width 0.25) (layer F.Cu) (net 16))
 (segment (start 109.314999 72.992999) (end 110.236 73.914) (width 0.25) (layer F.Cu) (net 16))
 (segment (start 110.236 73.914) (end 110.236 76.932803) (width 0.25) (layer F.Cu) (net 16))
 (segment (start 105.41 86.427919) (end 104.775 85.792919) (width 0.25) (layer F.Cu) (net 14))
 (segment (start 105.41 87.63) (end 105.41 86.427919) (width 0.25) (layer F.Cu) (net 14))
 (segment (start 104.775 85.792919) (end 104.775 82.55141) (width 0.25) (layer F.Cu) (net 14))
 (segment (start 100.095 77.87141) (end 104.775 82.55141) (width 0.25) (layer F.Cu) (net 14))
 (segment (start 100.095 76.41) (end 100.095 77.87141) (width 0.25) (layer F.Cu) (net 14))
 (segment (start 102.87 74.93) (end 102.87 76.708) (width 0.25) (layer F.Cu) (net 14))
 (segment (start 102.616 74.676) (end 102.87 74.93) (width 0.25) (layer F.Cu) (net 14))
 (segment (start 100.704 74.676) (end 102.616 74.676) (width 0.25) (layer F.Cu) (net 14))
 (segment (start 100.095 76.41) (end 100.095 75.285) (width 0.25) (layer F.Cu) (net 14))
 (segment (start 100.095 75.285) (end 100.704 74.676) (width 0.25) (layer F.Cu) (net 14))
 (segment (start 102.87 74.93) (end 100.33 72.39) (width 0.25) (layer B.Cu) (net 14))
 (segment (start 102.87 76.708) (end 102.87 74.93) (width 0.25) (layer B.Cu) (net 14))
 (segment (start 88.265 73.592081) (end 88.265 72.39) (width 0.25) (layer F.Cu) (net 6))
 (segment (start 88.265 77.155) (end 88.265 73.592081) (width 0.25) (layer F.Cu) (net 6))
 (segment (start 93.595 82.485) (end 88.265 77.155) (width 0.25) (layer F.Cu) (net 6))
 (segment (start 93.595 83.61) (end 93.595 82.485) (width 0.25) (layer F.Cu) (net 6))
 (segment (start 90.301612 84.281612) (end 89.84 83.82) (width 0.25) (layer F.Cu) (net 6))
 (segment (start 90.830001 84.810001) (end 90.301612 84.281612) (width 0.25) (layer F.Cu) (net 6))
 (segment (start 93.519999 84.810001) (end 90.830001 84.810001) (width 0.25) (layer F.Cu) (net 6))
 (segment (start 93.595 84.735) (end 93.519999 84.810001) (width 0.25) (layer F.Cu) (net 6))
 (segment (start 93.595 83.61) (end 93.595 84.735) (width 0.25) (layer F.Cu) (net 6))
 (segment (start 100.745 77.885) (end 100.745 76.41) (width 0.25) (layer F.Cu) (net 13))
 (segment (start 105.22501 82.36501) (end 100.745 77.885) (width 0.25) (layer F.Cu) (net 13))
 (segment (start 107.95 87.63) (end 105.22501 84.90501) (width 0.25) (layer F.Cu) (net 13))
 (segment (start 105.22501 84.90501) (end 105.22501 82.36501) (width 0.25) (layer F.Cu) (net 13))
 (segment (start 107.492504 75.84399) (end 106.40101 75.84399) (width 0.25) (layer F.Cu) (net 13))
 (segment (start 107.95 72.39) (end 107.95 75.386494) (width 0.25) (layer F.Cu) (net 13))
 (segment (start 107.95 75.386494) (end 107.492504 75.84399) (width 0.25) (layer F.Cu) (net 13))
 (segment (start 106.26099 75.98401) (end 106.26099 83.40099) (width 0.25) (layer F.Cu) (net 13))
 (segment (start 106.40101 75.84399) (end 106.26099 75.98401) (width 0.25) (layer F.Cu) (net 13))
 (segment (start 107.95 86.427919) (end 107.95 87.63) (width 0.25) (layer F.Cu) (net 13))
 (segment (start 107.95 84.151006) (end 107.95 86.427919) (width 0.25) (layer F.Cu) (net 13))
 (segment (start 107.492504 83.69351) (end 107.95 84.151006) (width 0.25) (layer F.Cu) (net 13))
 (segment (start 106.55351 83.69351) (end 107.492504 83.69351) (width 0.25) (layer F.Cu) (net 13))
 (segment (start 106.26099 83.40099) (end 106.55351 83.69351) (width 0.25) (layer F.Cu) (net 13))
 (segment (start 99.445 77.535) (end 99.445 76.41) (width 0.25) (layer F.Cu) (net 15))
 (segment (start 99.445 77.85782) (end 99.445 77.535) (width 0.25) (layer F.Cu) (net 15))
 (segment (start 102.87 81.28282) (end 99.445 77.85782) (width 0.25) (layer F.Cu) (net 15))
 (segment (start 102.87 87.63) (end 102.87 81.28282) (width 0.25) (layer F.Cu) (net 15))
 (segment (start 96.940001 73.239999) (end 97.79 72.39) (width 0.25) (layer F.Cu) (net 18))
 (segment (start 95.545 74.635) (end 96.940001 73.239999) (width 0.25) (layer F.Cu) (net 18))
 (segment (start 95.545 76.41) (end 95.545 74.635) (width 0.25) (layer F.Cu) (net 18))
 (segment (start 94.895 72.745) (end 95.25 72.39) (width 0.25) (layer F.Cu) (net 19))
 (segment (start 94.895 76.41) (end 94.895 72.745) (width 0.25) (layer F.Cu) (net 19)))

